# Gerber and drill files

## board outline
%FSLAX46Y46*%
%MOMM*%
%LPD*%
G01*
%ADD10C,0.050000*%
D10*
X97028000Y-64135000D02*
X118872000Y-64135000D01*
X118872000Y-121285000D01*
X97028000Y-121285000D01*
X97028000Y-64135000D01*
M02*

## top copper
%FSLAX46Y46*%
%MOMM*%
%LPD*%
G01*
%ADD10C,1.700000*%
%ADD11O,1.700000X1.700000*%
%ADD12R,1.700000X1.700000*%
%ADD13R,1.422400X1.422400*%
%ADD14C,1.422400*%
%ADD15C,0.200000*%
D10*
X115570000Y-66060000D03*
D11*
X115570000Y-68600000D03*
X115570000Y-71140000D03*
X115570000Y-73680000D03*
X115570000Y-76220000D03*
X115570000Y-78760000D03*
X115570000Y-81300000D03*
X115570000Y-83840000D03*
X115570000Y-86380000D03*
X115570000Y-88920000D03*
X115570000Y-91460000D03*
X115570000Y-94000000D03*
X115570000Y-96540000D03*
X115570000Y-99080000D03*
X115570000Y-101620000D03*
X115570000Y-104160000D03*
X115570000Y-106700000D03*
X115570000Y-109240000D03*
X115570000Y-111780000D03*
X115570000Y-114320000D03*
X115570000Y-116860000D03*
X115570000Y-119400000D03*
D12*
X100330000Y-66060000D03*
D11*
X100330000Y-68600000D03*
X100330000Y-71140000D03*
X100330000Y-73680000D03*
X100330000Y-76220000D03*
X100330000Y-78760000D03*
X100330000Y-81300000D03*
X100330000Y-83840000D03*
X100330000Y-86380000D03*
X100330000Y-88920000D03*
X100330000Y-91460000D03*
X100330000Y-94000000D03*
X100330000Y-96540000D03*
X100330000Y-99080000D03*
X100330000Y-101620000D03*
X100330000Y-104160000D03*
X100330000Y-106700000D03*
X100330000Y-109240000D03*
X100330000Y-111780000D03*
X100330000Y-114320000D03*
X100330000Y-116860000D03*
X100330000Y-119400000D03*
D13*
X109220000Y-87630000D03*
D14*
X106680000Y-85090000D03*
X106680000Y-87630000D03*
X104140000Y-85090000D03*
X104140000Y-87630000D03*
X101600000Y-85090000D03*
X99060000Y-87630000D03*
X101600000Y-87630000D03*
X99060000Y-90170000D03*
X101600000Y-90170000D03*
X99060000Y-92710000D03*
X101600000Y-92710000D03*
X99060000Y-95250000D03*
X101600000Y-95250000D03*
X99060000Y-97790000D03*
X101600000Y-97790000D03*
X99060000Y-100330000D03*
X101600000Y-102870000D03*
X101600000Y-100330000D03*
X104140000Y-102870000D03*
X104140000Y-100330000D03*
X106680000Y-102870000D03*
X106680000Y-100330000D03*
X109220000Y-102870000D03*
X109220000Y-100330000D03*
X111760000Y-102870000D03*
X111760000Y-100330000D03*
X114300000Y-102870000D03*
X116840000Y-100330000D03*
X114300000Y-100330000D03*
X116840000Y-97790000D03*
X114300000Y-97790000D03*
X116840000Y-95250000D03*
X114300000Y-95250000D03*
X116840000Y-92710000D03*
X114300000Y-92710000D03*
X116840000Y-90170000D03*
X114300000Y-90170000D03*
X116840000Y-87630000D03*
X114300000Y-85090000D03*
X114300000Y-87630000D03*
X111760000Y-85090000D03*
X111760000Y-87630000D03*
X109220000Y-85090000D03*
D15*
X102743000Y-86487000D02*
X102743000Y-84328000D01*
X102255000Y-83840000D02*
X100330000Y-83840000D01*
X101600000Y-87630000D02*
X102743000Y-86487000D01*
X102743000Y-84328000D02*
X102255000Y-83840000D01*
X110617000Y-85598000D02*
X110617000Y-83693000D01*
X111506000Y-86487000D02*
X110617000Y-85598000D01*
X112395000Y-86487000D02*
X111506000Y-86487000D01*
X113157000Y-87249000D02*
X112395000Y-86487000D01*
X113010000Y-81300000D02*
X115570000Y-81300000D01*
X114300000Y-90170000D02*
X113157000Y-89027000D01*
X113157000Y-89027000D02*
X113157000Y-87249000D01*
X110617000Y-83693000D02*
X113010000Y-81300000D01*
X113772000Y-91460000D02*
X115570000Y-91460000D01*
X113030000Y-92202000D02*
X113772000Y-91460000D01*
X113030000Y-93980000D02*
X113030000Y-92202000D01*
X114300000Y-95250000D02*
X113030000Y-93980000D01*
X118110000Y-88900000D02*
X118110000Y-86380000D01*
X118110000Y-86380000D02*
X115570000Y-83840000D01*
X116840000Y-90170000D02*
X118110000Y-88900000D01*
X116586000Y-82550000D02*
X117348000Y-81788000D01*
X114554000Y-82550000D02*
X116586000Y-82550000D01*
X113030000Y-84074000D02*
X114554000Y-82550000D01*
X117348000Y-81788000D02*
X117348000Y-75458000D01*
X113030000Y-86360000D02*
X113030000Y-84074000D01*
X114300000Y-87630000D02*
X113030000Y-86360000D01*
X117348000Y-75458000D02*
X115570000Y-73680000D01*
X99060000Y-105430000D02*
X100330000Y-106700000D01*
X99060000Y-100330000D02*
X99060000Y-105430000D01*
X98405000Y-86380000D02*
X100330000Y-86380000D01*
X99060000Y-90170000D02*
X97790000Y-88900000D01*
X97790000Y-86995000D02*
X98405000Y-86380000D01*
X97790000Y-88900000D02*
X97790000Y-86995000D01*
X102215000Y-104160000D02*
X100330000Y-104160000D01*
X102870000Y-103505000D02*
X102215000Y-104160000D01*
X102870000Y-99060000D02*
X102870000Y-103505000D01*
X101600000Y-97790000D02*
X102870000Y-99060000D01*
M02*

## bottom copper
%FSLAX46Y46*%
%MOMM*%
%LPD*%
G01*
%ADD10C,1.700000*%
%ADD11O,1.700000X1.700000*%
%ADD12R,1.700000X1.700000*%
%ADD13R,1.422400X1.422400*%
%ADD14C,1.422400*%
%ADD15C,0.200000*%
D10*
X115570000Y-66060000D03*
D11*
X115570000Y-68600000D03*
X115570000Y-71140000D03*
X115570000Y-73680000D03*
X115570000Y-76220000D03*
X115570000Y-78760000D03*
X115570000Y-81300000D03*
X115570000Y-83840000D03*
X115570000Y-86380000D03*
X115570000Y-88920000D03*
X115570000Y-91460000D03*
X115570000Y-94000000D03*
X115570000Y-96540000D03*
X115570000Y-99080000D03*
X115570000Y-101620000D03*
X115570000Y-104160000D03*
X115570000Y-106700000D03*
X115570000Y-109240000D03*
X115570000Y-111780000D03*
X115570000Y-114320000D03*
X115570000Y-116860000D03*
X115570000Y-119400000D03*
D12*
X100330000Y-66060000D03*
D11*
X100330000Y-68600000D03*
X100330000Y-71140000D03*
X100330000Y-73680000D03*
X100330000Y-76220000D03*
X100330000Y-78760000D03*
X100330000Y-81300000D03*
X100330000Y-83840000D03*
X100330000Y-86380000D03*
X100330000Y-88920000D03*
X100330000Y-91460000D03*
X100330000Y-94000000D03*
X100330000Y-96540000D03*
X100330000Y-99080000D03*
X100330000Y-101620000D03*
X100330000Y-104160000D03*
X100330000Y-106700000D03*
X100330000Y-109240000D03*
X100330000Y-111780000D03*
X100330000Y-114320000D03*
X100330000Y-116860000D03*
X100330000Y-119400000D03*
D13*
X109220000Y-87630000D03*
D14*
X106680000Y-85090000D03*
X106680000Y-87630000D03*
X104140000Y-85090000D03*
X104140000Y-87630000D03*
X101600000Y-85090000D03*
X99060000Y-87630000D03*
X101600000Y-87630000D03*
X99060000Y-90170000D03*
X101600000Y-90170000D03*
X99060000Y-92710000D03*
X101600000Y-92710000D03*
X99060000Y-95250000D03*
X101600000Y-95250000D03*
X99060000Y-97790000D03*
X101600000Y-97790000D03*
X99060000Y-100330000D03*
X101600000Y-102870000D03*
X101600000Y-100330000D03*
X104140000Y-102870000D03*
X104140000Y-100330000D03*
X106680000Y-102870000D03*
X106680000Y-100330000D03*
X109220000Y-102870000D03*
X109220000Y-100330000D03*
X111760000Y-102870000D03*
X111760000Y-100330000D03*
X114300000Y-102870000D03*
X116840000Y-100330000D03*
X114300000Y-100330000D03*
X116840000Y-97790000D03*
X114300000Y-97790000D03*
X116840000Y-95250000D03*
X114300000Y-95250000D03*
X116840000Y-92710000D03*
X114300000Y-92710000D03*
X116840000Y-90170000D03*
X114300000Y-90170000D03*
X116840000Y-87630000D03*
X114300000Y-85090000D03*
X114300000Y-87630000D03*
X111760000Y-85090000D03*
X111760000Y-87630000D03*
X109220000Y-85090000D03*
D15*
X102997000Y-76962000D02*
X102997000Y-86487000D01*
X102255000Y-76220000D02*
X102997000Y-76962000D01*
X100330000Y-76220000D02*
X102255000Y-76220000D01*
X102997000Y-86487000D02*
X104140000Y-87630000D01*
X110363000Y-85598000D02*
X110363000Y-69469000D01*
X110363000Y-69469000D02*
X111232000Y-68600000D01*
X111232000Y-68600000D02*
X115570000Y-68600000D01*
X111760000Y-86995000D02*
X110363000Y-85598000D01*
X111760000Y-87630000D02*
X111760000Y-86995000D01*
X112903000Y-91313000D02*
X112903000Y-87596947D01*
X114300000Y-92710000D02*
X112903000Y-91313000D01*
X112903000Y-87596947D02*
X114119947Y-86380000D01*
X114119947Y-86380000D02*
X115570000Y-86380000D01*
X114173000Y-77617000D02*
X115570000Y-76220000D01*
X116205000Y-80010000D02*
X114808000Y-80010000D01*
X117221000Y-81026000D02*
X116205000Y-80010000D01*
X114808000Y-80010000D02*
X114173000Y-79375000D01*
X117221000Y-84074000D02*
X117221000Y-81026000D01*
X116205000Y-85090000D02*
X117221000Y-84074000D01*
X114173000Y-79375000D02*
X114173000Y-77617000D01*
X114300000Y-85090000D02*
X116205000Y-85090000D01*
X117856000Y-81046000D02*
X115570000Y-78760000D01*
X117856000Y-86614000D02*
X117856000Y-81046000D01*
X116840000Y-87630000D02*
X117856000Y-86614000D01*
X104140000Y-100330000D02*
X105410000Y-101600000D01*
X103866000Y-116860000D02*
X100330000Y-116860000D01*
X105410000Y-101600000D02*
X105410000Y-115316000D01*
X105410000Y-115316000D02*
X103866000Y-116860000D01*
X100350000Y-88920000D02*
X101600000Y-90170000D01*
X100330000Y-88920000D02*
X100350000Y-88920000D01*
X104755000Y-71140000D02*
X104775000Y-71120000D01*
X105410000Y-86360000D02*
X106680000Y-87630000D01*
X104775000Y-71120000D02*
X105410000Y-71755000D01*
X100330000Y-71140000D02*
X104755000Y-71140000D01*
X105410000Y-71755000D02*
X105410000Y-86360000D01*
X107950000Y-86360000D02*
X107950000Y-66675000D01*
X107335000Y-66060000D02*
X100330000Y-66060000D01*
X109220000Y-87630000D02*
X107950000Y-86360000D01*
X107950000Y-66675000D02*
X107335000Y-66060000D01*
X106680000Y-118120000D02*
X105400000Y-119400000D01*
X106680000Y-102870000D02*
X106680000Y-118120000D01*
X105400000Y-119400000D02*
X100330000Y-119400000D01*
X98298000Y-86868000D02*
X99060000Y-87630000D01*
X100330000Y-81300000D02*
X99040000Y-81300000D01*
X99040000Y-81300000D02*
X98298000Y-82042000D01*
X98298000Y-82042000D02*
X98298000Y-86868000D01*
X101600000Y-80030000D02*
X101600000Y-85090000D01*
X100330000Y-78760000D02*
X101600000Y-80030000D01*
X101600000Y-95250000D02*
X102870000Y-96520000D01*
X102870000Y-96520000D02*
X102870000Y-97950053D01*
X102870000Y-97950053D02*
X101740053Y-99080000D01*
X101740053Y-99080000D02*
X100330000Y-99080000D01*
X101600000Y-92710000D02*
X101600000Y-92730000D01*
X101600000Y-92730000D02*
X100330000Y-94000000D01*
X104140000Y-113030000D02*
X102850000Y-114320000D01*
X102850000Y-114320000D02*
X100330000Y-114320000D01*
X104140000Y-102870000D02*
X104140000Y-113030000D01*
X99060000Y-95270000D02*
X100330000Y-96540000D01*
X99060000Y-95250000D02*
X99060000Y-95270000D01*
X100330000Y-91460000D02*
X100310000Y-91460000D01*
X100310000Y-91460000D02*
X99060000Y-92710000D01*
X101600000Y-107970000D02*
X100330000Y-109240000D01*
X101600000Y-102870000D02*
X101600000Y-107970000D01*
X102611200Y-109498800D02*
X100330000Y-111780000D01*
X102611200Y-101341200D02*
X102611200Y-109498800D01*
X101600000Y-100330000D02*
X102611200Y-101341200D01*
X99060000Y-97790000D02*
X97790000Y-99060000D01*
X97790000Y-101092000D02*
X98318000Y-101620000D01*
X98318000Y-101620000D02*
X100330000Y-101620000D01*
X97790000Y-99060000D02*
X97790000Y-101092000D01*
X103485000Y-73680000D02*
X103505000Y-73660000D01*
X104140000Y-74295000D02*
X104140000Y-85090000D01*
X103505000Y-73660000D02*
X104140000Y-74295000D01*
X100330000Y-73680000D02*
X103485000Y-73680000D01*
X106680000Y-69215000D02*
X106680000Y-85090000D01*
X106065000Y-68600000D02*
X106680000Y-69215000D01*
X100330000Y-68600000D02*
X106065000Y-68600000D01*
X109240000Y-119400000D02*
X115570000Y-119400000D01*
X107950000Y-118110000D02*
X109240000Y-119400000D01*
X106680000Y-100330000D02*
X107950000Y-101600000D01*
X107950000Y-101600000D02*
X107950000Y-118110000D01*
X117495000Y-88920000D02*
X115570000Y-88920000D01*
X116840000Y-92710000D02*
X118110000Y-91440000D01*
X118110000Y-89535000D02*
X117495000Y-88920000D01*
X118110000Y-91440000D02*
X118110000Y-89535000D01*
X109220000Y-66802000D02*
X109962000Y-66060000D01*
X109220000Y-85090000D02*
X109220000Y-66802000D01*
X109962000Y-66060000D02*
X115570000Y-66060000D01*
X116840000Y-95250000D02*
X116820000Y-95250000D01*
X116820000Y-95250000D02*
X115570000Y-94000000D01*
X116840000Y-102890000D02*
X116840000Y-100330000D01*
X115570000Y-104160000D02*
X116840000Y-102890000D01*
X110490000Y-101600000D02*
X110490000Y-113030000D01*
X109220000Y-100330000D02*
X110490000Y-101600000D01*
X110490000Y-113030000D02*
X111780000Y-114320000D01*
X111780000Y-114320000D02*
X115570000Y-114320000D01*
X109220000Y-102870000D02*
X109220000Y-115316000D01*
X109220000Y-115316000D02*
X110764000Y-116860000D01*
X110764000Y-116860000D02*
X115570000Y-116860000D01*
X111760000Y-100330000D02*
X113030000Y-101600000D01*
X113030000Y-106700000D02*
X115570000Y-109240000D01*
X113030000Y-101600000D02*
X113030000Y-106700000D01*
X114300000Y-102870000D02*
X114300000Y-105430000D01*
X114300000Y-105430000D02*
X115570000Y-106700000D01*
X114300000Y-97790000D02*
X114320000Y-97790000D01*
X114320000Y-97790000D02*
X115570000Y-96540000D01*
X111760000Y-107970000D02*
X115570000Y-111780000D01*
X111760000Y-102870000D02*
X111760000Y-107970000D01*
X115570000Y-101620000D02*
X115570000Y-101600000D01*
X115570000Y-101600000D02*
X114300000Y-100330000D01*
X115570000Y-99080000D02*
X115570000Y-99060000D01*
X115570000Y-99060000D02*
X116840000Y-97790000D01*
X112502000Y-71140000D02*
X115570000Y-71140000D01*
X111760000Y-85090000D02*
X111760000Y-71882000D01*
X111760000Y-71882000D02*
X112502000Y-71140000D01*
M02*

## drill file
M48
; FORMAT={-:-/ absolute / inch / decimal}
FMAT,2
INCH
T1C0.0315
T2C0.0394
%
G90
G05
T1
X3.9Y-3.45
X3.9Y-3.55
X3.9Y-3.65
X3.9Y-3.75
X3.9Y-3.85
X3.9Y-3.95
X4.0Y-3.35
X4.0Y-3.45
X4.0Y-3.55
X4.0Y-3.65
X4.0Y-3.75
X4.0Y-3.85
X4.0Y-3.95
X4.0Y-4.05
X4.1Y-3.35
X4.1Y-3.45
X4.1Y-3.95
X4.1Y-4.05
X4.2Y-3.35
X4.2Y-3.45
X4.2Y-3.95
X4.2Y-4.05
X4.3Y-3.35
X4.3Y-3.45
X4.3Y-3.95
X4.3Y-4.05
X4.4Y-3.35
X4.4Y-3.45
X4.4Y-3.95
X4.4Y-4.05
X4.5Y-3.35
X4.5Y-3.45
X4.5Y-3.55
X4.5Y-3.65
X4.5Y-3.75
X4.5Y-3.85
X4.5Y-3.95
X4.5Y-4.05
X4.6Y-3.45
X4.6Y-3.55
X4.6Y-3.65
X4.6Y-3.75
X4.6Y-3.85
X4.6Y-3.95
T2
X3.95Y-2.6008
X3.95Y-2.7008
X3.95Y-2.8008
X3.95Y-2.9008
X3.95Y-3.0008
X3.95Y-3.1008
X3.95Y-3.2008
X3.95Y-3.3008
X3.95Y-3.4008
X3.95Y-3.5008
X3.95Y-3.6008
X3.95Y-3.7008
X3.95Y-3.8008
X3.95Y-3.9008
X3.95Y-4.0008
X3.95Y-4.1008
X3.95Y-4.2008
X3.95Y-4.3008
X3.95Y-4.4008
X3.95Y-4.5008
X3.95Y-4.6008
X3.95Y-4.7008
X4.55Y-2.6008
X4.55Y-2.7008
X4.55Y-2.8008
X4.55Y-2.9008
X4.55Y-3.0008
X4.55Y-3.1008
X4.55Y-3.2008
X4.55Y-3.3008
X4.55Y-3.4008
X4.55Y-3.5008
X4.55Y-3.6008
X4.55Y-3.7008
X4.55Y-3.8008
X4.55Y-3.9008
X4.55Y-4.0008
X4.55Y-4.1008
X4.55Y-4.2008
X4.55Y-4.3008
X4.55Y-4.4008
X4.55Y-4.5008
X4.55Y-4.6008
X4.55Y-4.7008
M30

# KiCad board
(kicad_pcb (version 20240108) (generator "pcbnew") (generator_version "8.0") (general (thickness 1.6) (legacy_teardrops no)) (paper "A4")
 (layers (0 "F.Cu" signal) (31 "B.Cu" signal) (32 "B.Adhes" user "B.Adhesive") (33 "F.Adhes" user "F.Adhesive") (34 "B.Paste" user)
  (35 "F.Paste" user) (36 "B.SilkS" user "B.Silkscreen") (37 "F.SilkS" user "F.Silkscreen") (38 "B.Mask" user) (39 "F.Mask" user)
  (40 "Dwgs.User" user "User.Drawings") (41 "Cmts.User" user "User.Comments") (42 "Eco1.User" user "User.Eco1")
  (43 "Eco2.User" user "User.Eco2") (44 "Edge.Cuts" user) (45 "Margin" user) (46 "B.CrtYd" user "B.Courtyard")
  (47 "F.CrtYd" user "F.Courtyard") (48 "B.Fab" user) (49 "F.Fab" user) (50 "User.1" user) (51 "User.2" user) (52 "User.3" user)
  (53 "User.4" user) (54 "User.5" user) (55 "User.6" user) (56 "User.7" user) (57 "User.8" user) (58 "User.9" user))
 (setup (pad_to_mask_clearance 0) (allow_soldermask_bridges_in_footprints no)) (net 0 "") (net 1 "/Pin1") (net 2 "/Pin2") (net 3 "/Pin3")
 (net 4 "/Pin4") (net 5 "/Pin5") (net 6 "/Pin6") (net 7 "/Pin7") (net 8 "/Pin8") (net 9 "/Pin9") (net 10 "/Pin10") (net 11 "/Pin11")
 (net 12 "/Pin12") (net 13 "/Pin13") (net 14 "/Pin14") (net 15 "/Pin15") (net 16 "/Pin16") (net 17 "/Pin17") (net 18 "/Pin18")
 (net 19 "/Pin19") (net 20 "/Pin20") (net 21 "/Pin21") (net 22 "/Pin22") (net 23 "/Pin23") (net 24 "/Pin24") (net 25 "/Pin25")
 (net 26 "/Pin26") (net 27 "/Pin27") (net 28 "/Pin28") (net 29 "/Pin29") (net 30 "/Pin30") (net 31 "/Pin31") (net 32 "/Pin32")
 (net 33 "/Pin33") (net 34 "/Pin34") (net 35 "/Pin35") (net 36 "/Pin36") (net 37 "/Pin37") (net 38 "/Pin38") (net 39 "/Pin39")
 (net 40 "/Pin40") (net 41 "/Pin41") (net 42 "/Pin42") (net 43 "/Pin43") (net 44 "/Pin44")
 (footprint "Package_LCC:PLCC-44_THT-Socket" (layer "F.Cu") (at 109.22 87.63)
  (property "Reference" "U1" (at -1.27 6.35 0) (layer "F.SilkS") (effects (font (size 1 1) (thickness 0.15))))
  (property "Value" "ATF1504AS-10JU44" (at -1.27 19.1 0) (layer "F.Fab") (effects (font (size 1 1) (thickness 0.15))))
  (pad "1" thru_hole rect (at 0 0) (size 1.4224 1.4224) (drill 0.8) (layers "*.Cu" "*.Mask") (remove_unused_layers no) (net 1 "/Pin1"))
  (pad "2" thru_hole circle (at -2.54 -2.54) (size 1.4224 1.4224) (drill 0.8) (layers "*.Cu" "*.Mask") (remove_unused_layers no)
   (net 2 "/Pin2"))
  (pad "3" thru_hole circle (at -2.54 0) (size 1.4224 1.4224) (drill 0.8) (layers "*.Cu" "*.Mask") (remove_unused_layers no) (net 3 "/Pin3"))
  (pad "4" thru_hole circle (at -5.08 -2.54) (size 1.4224 1.4224) (drill 0.8) (layers "*.Cu" "*.Mask") (remove_unused_layers no)
   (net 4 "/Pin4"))
  (pad "5" thru_hole circle (at -5.08 0) (size 1.4224 1.4224) (drill 0.8) (layers "*.Cu" "*.Mask") (remove_unused_layers no) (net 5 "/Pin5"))
  (pad "6" thru_hole circle (at -7.62 -2.54) (size 1.4224 1.4224) (drill 0.8) (layers "*.Cu" "*.Mask") (remove_unused_layers no)
   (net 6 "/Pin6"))
  (pad "7" thru_hole circle (at -10.16 0) (size 1.4224 1.4224) (drill 0.8) (layers "*.Cu" "*.Mask") (remove_unused_layers no)
   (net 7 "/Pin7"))
  (pad "8" thru_hole circle (at -7.62 0) (size 1.4224 1.4224) (drill 0.8) (layers "*.Cu" "*.Mask") (remove_unused_layers no) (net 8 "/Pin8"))
  (pad "9" thru_hole circle (at -10.16 2.54) (size 1.4224 1.4224) (drill 0.8) (layers "*.Cu" "*.Mask") (remove_unused_layers no)
   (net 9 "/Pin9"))
  (pad "10" thru_hole circle (at -7.62 2.54) (size 1.4224 1.4224) (drill 0.8) (layers "*.Cu" "*.Mask") (remove_unused_layers no)
   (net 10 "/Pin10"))
  (pad "11" thru_hole circle (at -10.16 5.08) (size 1.4224 1.4224) (drill 0.8) (layers "*.Cu" "*.Mask") (remove_unused_layers no)
   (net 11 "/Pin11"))
  (pad "12" thru_hole circle (at -7.62 5.08) (size 1.4224 1.4224) (drill 0.8) (layers "*.Cu" "*.Mask") (remove_unused_layers no)
   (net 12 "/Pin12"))
  (pad "13" thru_hole circle (at -10.16 7.62) (size 1.4224 1.4224) (drill 0.8) (layers "*.Cu" "*.Mask") (remove_unused_layers no)
   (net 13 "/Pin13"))
  (pad "14" thru_hole circle (at -7.62 7.62) (size 1.4224 1.4224) (drill 0.8) (layers "*.Cu" "*.Mask") (remove_unused_layers no)
   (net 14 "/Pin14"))
  (pad "15" thru_hole circle (at -10.16 10.16) (size 1.4224 1.4224) (drill 0.8) (layers "*.Cu" "*.Mask") (remove_unused_layers no)
   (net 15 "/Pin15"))
  (pad "16" thru_hole circle (at -7.62 10.16) (size 1.4224 1.4224) (drill 0.8) (layers "*.Cu" "*.Mask") (remove_unused_layers no)
   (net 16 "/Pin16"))
  (pad "17" thru_hole circle (at -10.16 12.7) (size 1.4224 1.4224) (drill 0.8) (layers "*.Cu" "*.Mask") (remove_unused_layers no)
   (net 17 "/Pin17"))
  (pad "18" thru_hole circle (at -7.62 15.24) (size 1.4224 1.4224) (drill 0.8) (layers "*.Cu" "*.Mask") (remove_unused_layers no)
   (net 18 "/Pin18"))
  (pad "19" thru_hole circle (at -7.62 12.7) (size 1.4224 1.4224) (drill 0.8) (layers "*.Cu" "*.Mask") (remove_unused_layers no)
   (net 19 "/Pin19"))
  (pad "20" thru_hole circle (at -5.08 15.24) (size 1.4224 1.4224) (drill 0.8) (layers "*.Cu" "*.Mask") (remove_unused_layers no)
   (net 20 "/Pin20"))
  (pad "21" thru_hole circle (at -5.08 12.7) (size 1.4224 1.4224) (drill 0.8) (layers "*.Cu" "*.Mask") (remove_unused_layers no)
   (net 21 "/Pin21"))
  (pad "22" thru_hole circle (at -2.54 15.24) (size 1.4224 1.4224) (drill 0.8) (layers "*.Cu" "*.Mask") (remove_unused_layers no)
   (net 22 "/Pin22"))
  (pad "23" thru_hole circle (at -2.54 12.7) (size 1.4224 1.4224) (drill 0.8) (layers "*.Cu" "*.Mask") (remove_unused_layers no)
   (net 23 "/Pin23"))
  (pad "24" thru_hole circle (at 0 15.24) (size 1.4224 1.4224) (drill 0.8) (layers "*.Cu" "*.Mask") (remove_unused_layers no)
   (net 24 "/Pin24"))
  (pad "25" thru_hole circle (at 0 12.7) (size 1.4224 1.4224) (drill 0.8) (layers "*.Cu" "*.Mask") (remove_unused_layers no)
   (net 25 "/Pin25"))
  (pad "26" thru_hole circle (at 2.54 15.24) (size 1.4224 1.4224) (drill 0.8) (layers "*.Cu" "*.Mask") (remove_unused_layers no)
   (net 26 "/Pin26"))
  (pad "27" thru_hole circle (at 2.54 12.7) (size 1.4224 1.4224) (drill 0.8) (layers "*.Cu" "*.Mask") (remove_unused_layers no)
   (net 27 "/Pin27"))
  (pad "28" thru_hole circle (at 5.08 15.24) (size 1.4224 1.4224) (drill 0.8) (layers "*.Cu" "*.Mask") (remove_unused_layers no)
   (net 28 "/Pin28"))
  (pad "29" thru_hole circle (at 7.62 12.7) (size 1.4224 1.4224) (drill 0.8) (layers "*.Cu" "*.Mask") (remove_unused_layers no)
   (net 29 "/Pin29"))
  (pad "30" thru_hole circle (at 5.08 12.7) (size 1.4224 1.4224) (drill 0.8) (layers "*.Cu" "*.Mask") (remove_unused_layers no)
   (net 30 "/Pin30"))
  (pad "31" thru_hole circle (at 7.62 10.16) (size 1.4224 1.4224) (drill 0.8) (layers "*.Cu" "*.Mask") (remove_unused_layers no)
   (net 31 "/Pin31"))
  (pad "32" thru_hole circle (at 5.08 10.16) (size 1.4224 1.4224) (drill 0.8) (layers "*.Cu" "*.Mask") (remove_unused_layers no)
   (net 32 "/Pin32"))
  (pad "33" thru_hole circle (at 7.62 7.62) (size 1.4224 1.4224) (drill 0.8) (layers "*.Cu" "*.Mask") (remove_unused_layers no)
   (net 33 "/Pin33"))
  (pad "34" thru_hole circle (at 5.08 7.62) (size 1.4224 1.4224) (drill 0.8) (layers "*.Cu" "*.Mask") (remove_unused_layers no)
   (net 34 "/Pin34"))
  (pad "35" thru_hole circle (at 7.62 5.08) (size 1.4224 1.4224) (drill 0.8) (layers "*.Cu" "*.Mask") (remove_unused_layers no)
   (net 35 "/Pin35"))
  (pad "36" thru_hole circle (at 5.08 5.08) (size 1.4224 1.4224) (drill 0.8) (layers "*.Cu" "*.Mask") (remove_unused_layers no)
   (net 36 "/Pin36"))
  (pad "37" thru_hole circle (at 7.62 2.54) (size 1.4224 1.4224) (drill 0.8) (layers "*.Cu" "*.Mask") (remove_unused_layers no)
   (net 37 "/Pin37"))
  (pad "38" thru_hole circle (at 5.08 2.54) (size 1.4224 1.4224) (drill 0.8) (layers "*.Cu" "*.Mask") (remove_unused_layers no)
   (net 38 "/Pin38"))
  (pad "39" thru_hole circle (at 7.62 0) (size 1.4224 1.4224) (drill 0.8) (layers "*.Cu" "*.Mask") (remove_unused_layers no)
   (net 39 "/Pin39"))
  (pad "40" thru_hole circle (at 5.08 -2.54) (size 1.4224 1.4224) (drill 0.8) (layers "*.Cu" "*.Mask") (remove_unused_layers no)
   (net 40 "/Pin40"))
  (pad "41" thru_hole circle (at 5.08 0) (size 1.4224 1.4224) (drill 0.8) (layers "*.Cu" "*.Mask") (remove_unused_layers no)
   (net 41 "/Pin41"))
  (pad "42" thru_hole circle (at 2.54 -2.54) (size 1.4224 1.4224) (drill 0.8) (layers "*.Cu" "*.Mask") (remove_unused_layers no)
   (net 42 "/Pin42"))
  (pad "43" thru_hole circle (at 2.54 0) (size 1.4224 1.4224) (drill 0.8) (layers "*.Cu" "*.Mask") (remove_unused_layers no)
   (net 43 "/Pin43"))
  (pad "44" thru_hole circle (at 0 -2.54) (size 1.4224 1.4224) (drill 0.8) (layers "*.Cu" "*.Mask") (remove_unused_layers no)
   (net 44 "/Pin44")))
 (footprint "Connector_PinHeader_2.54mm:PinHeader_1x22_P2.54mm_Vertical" (layer "B.Cu") (at 115.57 66.06 180)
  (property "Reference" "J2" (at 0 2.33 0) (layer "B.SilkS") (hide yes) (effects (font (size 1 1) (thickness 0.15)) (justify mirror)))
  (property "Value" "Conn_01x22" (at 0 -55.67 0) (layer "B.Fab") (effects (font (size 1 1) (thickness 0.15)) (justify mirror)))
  (pad "1" thru_hole circle (at 0 0 180) (size 1.7 1.7) (drill 1) (layers "*.Cu" "*.Mask") (remove_unused_layers no) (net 44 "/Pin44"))
  (pad "2" thru_hole oval (at 0 -2.54 180) (size 1.7 1.7) (drill 1) (layers "*.Cu" "*.Mask") (remove_unused_layers no) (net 43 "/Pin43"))
  (pad "3" thru_hole oval (at 0 -5.08 180) (size 1.7 1.7) (drill 1) (layers "*.Cu" "*.Mask") (remove_unused_layers no) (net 42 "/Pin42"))
  (pad "4" thru_hole oval (at 0 -7.62 180) (size 1.7 1.7) (drill 1) (layers "*.Cu" "*.Mask") (remove_unused_layers no) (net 41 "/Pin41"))
  (pad "5" thru_hole oval (at 0 -10.16 180) (size 1.7 1.7) (drill 1) (layers "*.Cu" "*.Mask") (remove_unused_layers no) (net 40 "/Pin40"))
  (pad "6" thru_hole oval (at 0 -12.7 180) (size 1.7 1.7) (drill 1) (layers "*.Cu" "*.Mask") (remove_unused_layers no) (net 39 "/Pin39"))
  (pad "7" thru_hole oval (at 0 -15.24 180) (size 1.7 1.7) (drill 1) (layers "*.Cu" "*.Mask") (remove_unused_layers no) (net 38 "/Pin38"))
  (pad "8" thru_hole oval (at 0 -17.78 180) (size 1.7 1.7) (drill 1) (layers "*.Cu" "*.Mask") (remove_unused_layers no) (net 37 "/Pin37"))
  (pad "9" thru_hole oval (at 0 -20.32 180) (size 1.7 1.7) (drill 1) (layers "*.Cu" "*.Mask") (remove_unused_layers no) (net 36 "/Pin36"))
  (pad "10" thru_hole oval (at 0 -22.86 180) (size 1.7 1.7) (drill 1) (layers "*.Cu" "*.Mask") (remove_unused_layers no) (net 35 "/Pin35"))
  (pad "11" thru_hole oval (at 0 -25.4 180) (size 1.7 1.7) (drill 1) (layers "*.Cu" "*.Mask") (remove_unused_layers no) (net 34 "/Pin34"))
  (pad "12" thru_hole oval (at 0 -27.94 180) (size 1.7 1.7) (drill 1) (layers "*.Cu" "*.Mask") (remove_unused_layers no) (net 33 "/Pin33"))
  (pad "13" thru_hole oval (at 0 -30.48 180) (size 1.7 1.7) (drill 1) (layers "*.Cu" "*.Mask") (remove_unused_layers no) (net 32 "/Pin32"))
  (pad "14" thru_hole oval (at 0 -33.02 180) (size 1.7 1.7) (drill 1) (layers "*.Cu" "*.Mask") (remove_unused_layers no) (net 31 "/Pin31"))
  (pad "15" thru_hole oval (at 0 -35.56 180) (size 1.7 1.7) (drill 1) (layers "*.Cu" "*.Mask") (remove_unused_layers no) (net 30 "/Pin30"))
  (pad "16" thru_hole oval (at 0 -38.1 180) (size 1.7 1.7) (drill 1) (layers "*.Cu" "*.Mask") (remove_unused_layers no) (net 29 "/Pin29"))
  (pad "17" thru_hole oval (at 0 -40.64 180) (size 1.7 1.7) (drill 1) (layers "*.Cu" "*.Mask") (remove_unused_layers no) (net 28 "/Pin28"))
  (pad "18" thru_hole oval (at 0 -43.18 180) (size 1.7 1.7) (drill 1) (layers "*.Cu" "*.Mask") (remove_unused_layers no) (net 27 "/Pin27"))
  (pad "19" thru_hole oval (at 0 -45.72 180) (size 1.7 1.7) (drill 1) (layers "*.Cu" "*.Mask") (remove_unused_layers no) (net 26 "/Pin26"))
  (pad "20" thru_hole oval (at 0 -48.26 180) (size 1.7 1.7) (drill 1) (layers "*.Cu" "*.Mask") (remove_unused_layers no) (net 25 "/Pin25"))
  (pad "21" thru_hole oval (at 0 -50.8 180) (size 1.7 1.7) (drill 1) (layers "*.Cu" "*.Mask") (remove_unused_layers no) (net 24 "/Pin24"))
  (pad "22" thru_hole oval (at 0 -53.34 180) (size 1.7 1.7) (drill 1) (layers "*.Cu" "*.Mask") (remove_unused_layers no) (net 23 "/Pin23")))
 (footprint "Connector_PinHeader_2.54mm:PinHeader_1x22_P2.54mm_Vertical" (layer "B.Cu") (at 100.33 66.06 180)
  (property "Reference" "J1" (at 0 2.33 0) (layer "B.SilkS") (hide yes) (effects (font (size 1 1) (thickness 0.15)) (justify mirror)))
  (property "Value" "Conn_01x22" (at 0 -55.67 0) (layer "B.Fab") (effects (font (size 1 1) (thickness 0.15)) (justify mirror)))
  (pad "1" thru_hole rect (at 0 0 180) (size 1.7 1.7) (drill 1) (layers "*.Cu" "*.Mask") (remove_unused_layers no) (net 1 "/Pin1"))
  (pad "2" thru_hole oval (at 0 -2.54 180) (size 1.7 1.7) (drill 1) (layers "*.Cu" "*.Mask") (remove_unused_layers no) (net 2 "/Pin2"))
  (pad "3" thru_hole oval (at 0 -5.08 180) (size 1.7 1.7) (drill 1) (layers "*.Cu" "*.Mask") (remove_unused_layers no) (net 3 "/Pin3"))
  (pad "4" thru_hole oval (at 0 -7.62 180) (size 1.7 1.7) (drill 1) (layers "*.Cu" "*.Mask") (remove_unused_layers no) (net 4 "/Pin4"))
  (pad "5" thru_hole oval (at 0 -10.16 180) (size 1.7 1.7) (drill 1) (layers "*.Cu" "*.Mask") (remove_unused_layers no) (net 5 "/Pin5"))
  (pad "6" thru_hole oval (at 0 -12.7 180) (size 1.7 1.7) (drill 1) (layers "*.Cu" "*.Mask") (remove_unused_layers no) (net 6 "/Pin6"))
  (pad "7" thru_hole oval (at 0 -15.24 180) (size 1.7 1.7) (drill 1) (layers "*.Cu" "*.Mask") (remove_unused_layers no) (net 7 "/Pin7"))
  (pad "8" thru_hole oval (at 0 -17.78 180) (size 1.7 1.7) (drill 1) (layers "*.Cu" "*.Mask") (remove_unused_layers no) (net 8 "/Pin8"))
  (pad "9" thru_hole oval (at 0 -20.32 180) (size 1.7 1.7) (drill 1) (layers "*.Cu" "*.Mask") (remove_unused_layers no) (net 9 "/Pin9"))
  (pad "10" thru_hole oval (at 0 -22.86 180) (size 1.7 1.7) (drill 1) (layers "*.Cu" "*.Mask") (remove_unused_layers no) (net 10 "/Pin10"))
  (pad "11" thru_hole oval (at 0 -25.4 180) (size 1.7 1.7) (drill 1) (layers "*.Cu" "*.Mask") (remove_unused_layers no) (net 11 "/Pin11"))
  (pad "12" thru_hole oval (at 0 -27.94 180) (size 1.7 1.7) (drill 1) (layers "*.Cu" "*.Mask") (remove_unused_layers no) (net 12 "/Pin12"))
  (pad "13" thru_hole oval (at 0 -30.48 180) (size 1.7 1.7) (drill 1) (layers "*.Cu" "*.Mask") (remove_unused_layers no) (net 13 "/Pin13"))
  (pad "14" thru_hole oval (at 0 -33.02 180) (size 1.7 1.7) (drill 1) (layers "*.Cu" "*.Mask") (remove_unused_layers no) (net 14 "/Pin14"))
  (pad "15" thru_hole oval (at 0 -35.56 180) (size 1.7 1.7) (drill 1) (layers "*.Cu" "*.Mask") (remove_unused_layers no) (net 15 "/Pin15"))
  (pad "16" thru_hole oval (at 0 -38.1 180) (size 1.7 1.7) (drill 1) (layers "*.Cu" "*.Mask") (remove_unused_layers no) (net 16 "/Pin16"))
  (pad "17" thru_hole oval (at 0 -40.64 180) (size 1.7 1.7) (drill 1) (layers "*.Cu" "*.Mask") (remove_unused_layers no) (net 17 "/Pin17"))
  (pad "18" thru_hole oval (at 0 -43.18 180) (size 1.7 1.7) (drill 1) (layers "*.Cu" "*.Mask") (remove_unused_layers no) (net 18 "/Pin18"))
  (pad "19" thru_hole oval (at 0 -45.72 180) (size 1.7 1.7) (drill 1) (layers "*.Cu" "*.Mask") (remove_unused_layers no) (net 19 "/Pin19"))
  (pad "20" thru_hole oval (at 0 -48.26 180) (size 1.7 1.7) (drill 1) (layers "*.Cu" "*.Mask") (remove_unused_layers no) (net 20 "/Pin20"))
  (pad "21" thru_hole oval (at 0 -50.8 180) (size 1.7 1.7) (drill 1) (layers "*.Cu" "*.Mask") (remove_unused_layers no) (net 21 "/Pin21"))
  (pad "22" thru_hole oval (at 0 -53.34 180) (size 1.7 1.7) (drill 1) (layers "*.Cu" "*.Mask") (remove_unused_layers no) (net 22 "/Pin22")))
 (gr_rect (start 97.028 64.135) (end 118.872 121.285) (stroke (width 0.05) (type default)) (fill none) (layer "Edge.Cuts"))
 (segment (start 104.14 100.33) (end 105.41 101.6) (width 0.2) (layer "B.Cu") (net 21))
 (segment (start 103.866 116.86) (end 100.33 116.86) (width 0.2) (layer "B.Cu") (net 21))
 (segment (start 105.41 101.6) (end 105.41 115.316) (width 0.2) (layer "B.Cu") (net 21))
 (segment (start 105.41 115.316) (end 103.866 116.86) (width 0.2) (layer "B.Cu") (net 21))
 (segment (start 100.35 88.92) (end 101.6 90.17) (width 0.2) (layer "B.Cu") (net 10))
 (segment (start 100.33 88.92) (end 100.35 88.92) (width 0.2) (layer "B.Cu") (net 10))
 (segment (start 99.06 105.43) (end 100.33 106.7) (width 0.2) (layer "F.Cu") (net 17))
 (segment (start 99.06 100.33) (end 99.06 105.43) (width 0.2) (layer "F.Cu") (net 17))
 (segment (start 104.755 71.14) (end 104.775 71.12) (width 0.2) (layer "B.Cu") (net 3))
 (segment (start 105.41 86.36) (end 106.68 87.63) (width 0.2) (layer "B.Cu") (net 3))
 (segment (start 104.775 71.12) (end 105.41 71.755) (width 0.2) (layer "B.Cu") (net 3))
 (segment (start 100.33 71.14) (end 104.755 71.14) (width 0.2) (layer "B.Cu") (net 3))
 (segment (start 105.41 71.755) (end 105.41 86.36) (width 0.2) (layer "B.Cu") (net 3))
 (segment (start 107.95 86.36) (end 107.95 66.675) (width 0.2) (layer "B.Cu") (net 1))
 (segment (start 107.335 66.06) (end 100.33 66.06) (width 0.2) (layer "B.Cu") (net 1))
 (segment (start 109.22 87.63) (end 107.95 86.36) (width 0.2) (layer "B.Cu") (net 1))
 (segment (start 107.95 66.675) (end 107.335 66.06) (width 0.2) (layer "B.Cu") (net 1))
 (segment (start 106.68 118.12) (end 105.4 119.4) (width 0.2) (layer "B.Cu") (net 22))
 (segment (start 106.68 102.87) (end 106.68 118.12) (width 0.2) (layer "B.Cu") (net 22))
 (segment (start 105.4 119.4) (end 100.33 119.4) (width 0.2) (layer "B.Cu") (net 22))
 (segment (start 102.743 84.328) (end 102.255 83.84) (width 0.2) (layer "F.Cu") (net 8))
 (segment (start 101.6 87.63) (end 102.743 86.487) (width 0.2) (layer "F.Cu") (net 8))
 (segment (start 102.743 86.487) (end 102.743 84.328) (width 0.2) (layer "F.Cu") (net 8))
 (segment (start 102.255 83.84) (end 100.33 83.84) (width 0.2) (layer "F.Cu") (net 8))
 (segment (start 98.298 86.868) (end 99.06 87.63) (width 0.2) (layer "B.Cu") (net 7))
 (segment (start 100.33 81.3) (end 99.04 81.3) (width 0.2) (layer "B.Cu") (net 7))
 (segment (start 99.04 81.3) (end 98.298 82.042) (width 0.2) (layer "B.Cu") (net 7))
 (segment (start 98.298 82.042) (end 98.298 86.868) (width 0.2) (layer "B.Cu") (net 7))
 (segment (start 101.6 80.03) (end 101.6 85.09) (width 0.2) (layer "B.Cu") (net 6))
 (segment (start 100.33 78.76) (end 101.6 80.03) (width 0.2) (layer "B.Cu") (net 6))
 (segment (start 101.6 95.25) (end 102.87 96.52) (width 0.2) (layer "B.Cu") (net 14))
 (segment (start 102.87 96.52) (end 102.87 97.950053) (width 0.2) (layer "B.Cu") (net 14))
 (segment (start 102.87 97.950053) (end 101.740053 99.08) (width 0.2) (layer "B.Cu") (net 14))
 (segment (start 101.740053 99.08) (end 100.33 99.08) (width 0.2) (layer "B.Cu") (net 14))
 (segment (start 101.6 92.71) (end 101.6 92.73) (width 0.2) (layer "B.Cu") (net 12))
 (segment (start 101.6 92.73) (end 100.33 94) (width 0.2) (layer "B.Cu") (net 12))
 (segment (start 98.405 86.38) (end 100.33 86.38) (width 0.2) (layer "F.Cu") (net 9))
 (segment (start 99.06 90.17) (end 97.79 88.9) (width 0.2) (layer "F.Cu") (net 9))
 (segment (start 97.79 86.995) (end 98.405 86.38) (width 0.2) (layer "F.Cu") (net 9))
 (segment (start 97.79 88.9) (end 97.79 86.995) (width 0.2) (layer "F.Cu") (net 9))
 (segment (start 104.14 113.03) (end 102.85 114.32) (width 0.2) (layer "B.Cu") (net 20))
 (segment (start 102.85 114.32) (end 100.33 114.32) (width 0.2) (layer "B.Cu") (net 20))
 (segment (start 104.14 102.87) (end 104.14 113.03) (width 0.2) (layer "B.Cu") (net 20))
 (segment (start 99.06 95.27) (end 100.33 96.54) (width 0.2) (layer "B.Cu") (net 13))
 (segment (start 99.06 95.25) (end 99.06 95.27) (width 0.2) (layer "B.Cu") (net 13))
 (segment (start 100.33 91.46) (end 100.31 91.46) (width 0.2) (layer "B.Cu") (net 11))
 (segment (start 100.31 91.46) (end 99.06 92.71) (width 0.2) (layer "B.Cu") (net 11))
 (segment (start 100.33 76.22) (end 102.255 76.22) (width 0.2) (layer "B.Cu") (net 5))
 (segment (start 102.997 86.487) (end 104.14 87.63) (width 0.2) (layer "B.Cu") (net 5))
 (segment (start 102.255 76.22) (end 102.997 76.962) (width 0.2) (layer "B.Cu") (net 5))
 (segment (start 102.997 76.962) (end 102.997 86.487) (width 0.2) (layer "B.Cu") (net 5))
 (segment (start 101.6 107.97) (end 100.33 109.24) (width 0.2) (layer "B.Cu") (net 18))
 (segment (start 101.6 102.87) (end 101.6 107.97) (width 0.2) (layer "B.Cu") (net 18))
 (segment (start 102.6112 109.4988) (end 100.33 111.78) (width 0.2) (layer "B.Cu") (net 19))
 (segment (start 102.6112 101.3412) (end 102.6112 109.4988) (width 0.2) (layer "B.Cu") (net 19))
 (segment (start 101.6 100.33) (end 102.6112 101.3412) (width 0.2) (layer "B.Cu") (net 19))
 (segment (start 99.06 97.79) (end 97.79 99.06) (width 0.2) (layer "B.Cu") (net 15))
 (segment (start 97.79 101.092) (end 98.318 101.62) (width 0.2) (layer "B.Cu") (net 15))
 (segment (start 98.318 101.62) (end 100.33 101.62) (width 0.2) (layer "B.Cu") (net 15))
 (segment (start 97.79 99.06) (end 97.79 101.092) (width 0.2) (layer "B.Cu") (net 15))
 (segment (start 102.215 104.16) (end 100.33 104.16) (width 0.2) (layer "F.Cu") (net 16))
 (segment (start 102.87 103.505) (end 102.215 104.16) (width 0.2) (layer "F.Cu") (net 16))
 (segment (start 102.87 99.06) (end 102.87 103.505) (width 0.2) (layer "F.Cu") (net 16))
 (segment (start 101.6 97.79) (end 102.87 99.06) (width 0.2) (layer "F.Cu") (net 16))
 (segment (start 103.485 73.68) (end 103.505 73.66) (width 0.2) (layer "B.Cu") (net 4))
 (segment (start 104.14 74.295) (end 104.14 85.09) (width 0.2) (layer "B.Cu") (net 4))
 (segment (start 103.505 73.66) (end 104.14 74.295) (width 0.2) (layer "B.Cu") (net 4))
 (segment (start 100.33 73.68) (end 103.485 73.68) (width 0.2) (layer "B.Cu") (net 4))
 (segment (start 106.68 69.215) (end 106.68 85.09) (width 0.2) (layer "B.Cu") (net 2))
 (segment (start 106.065 68.6) (end 106.68 69.215) (width 0.2) (layer "B.Cu") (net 2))
 (segment (start 100.33 68.6) (end 106.065 68.6) (width 0.2) (layer "B.Cu") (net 2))
 (segment (start 113.772 91.46) (end 115.57 91.46) (width 0.2) (layer "F.Cu") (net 34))
 (segment (start 113.03 93.98) (end 113.03 92.202) (width 0.2) (layer "F.Cu") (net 34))
 (segment (start 113.03 92.202) (end 113.772 91.46) (width 0.2) (layer "F.Cu") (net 34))
 (segment (start 114.3 95.25) (end 113.03 93.98) (width 0.2) (layer "F.Cu") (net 34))
 (segment (start 113.01 81.3) (end 115.57 81.3) (width 0.2) (layer "F.Cu") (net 38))
 (segment (start 111.506 86.487) (end 110.617 85.598) (width 0.2) (layer "F.Cu") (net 38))
 (segment (start 110.617 85.598) (end 110.617 83.693) (width 0.2) (layer "F.Cu") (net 38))
 (segment (start 113.157 89.027) (end 113.157 87.249) (width 0.2) (layer "F.Cu") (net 38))
 (segment (start 112.395 86.487) (end 111.506 86.487) (width 0.2) (layer "F.Cu") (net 38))
 (segment (start 110.617 83.693) (end 113.01 81.3) (width 0.2) (layer "F.Cu") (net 38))
 (segment (start 114.3 90.17) (end 113.157 89.027) (width 0.2) (layer "F.Cu") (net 38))
 (segment (start 113.157 87.249) (end 112.395 86.487) (width 0.2) (layer "F.Cu") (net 38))
 (segment (start 109.24 119.4) (end 115.57 119.4) (width 0.2) (layer "B.Cu") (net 23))
 (segment (start 107.95 118.11) (end 109.24 119.4) (width 0.2) (layer "B.Cu") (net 23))
 (segment (start 106.68 100.33) (end 107.95 101.6) (width 0.2) (layer "B.Cu") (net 23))
 (segment (start 107.95 101.6) (end 107.95 118.11) (width 0.2) (layer "B.Cu") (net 23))
 (segment (start 117.495 88.92) (end 115.57 88.92) (width 0.2) (layer "B.Cu") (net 35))
 (segment (start 116.84 92.71) (end 118.11 91.44) (width 0.2) (layer "B.Cu") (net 35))
 (segment (start 118.11 89.535) (end 117.495 88.92) (width 0.2) (layer "B.Cu") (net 35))
 (segment (start 118.11 91.44) (end 118.11 89.535) (width 0.2) (layer "B.Cu") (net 35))
 (segment (start 109.22 66.802) (end 109.962 66.06) (width 0.2) (layer "B.Cu") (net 44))
 (segment (start 109.22 85.09) (end 109.22 66.802) (width 0.2) (layer "B.Cu") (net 44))
 (segment (start 109.962 66.06) (end 115.57 66.06) (width 0.2) (layer "B.Cu") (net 44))
 (segment (start 116.84 95.25) (end 116.82 95.25) (width 0.2) (layer "B.Cu") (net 33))
 (segment (start 116.82 95.25) (end 115.57 94) (width 0.2) (layer "B.Cu") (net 33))
 (segment (start 116.205 80.01) (end 114.808 80.01) (width 0.2) (layer "B.Cu") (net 40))
 (segment (start 117.221 81.026) (end 116.205 80.01) (width 0.2) (layer "B.Cu") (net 40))
 (segment (start 116.205 85.09) (end 117.221 84.074) (width 0.2) (layer "B.Cu") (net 40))
 (segment (start 114.808 80.01) (end 114.173 79.375) (width 0.2) (layer "B.Cu") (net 40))
 (segment (start 114.173 77.617) (end 115.57 76.22) (width 0.2) (layer "B.Cu") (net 40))
 (segment (start 114.3 85.09) (end 116.205 85.09) (width 0.2) (layer "B.Cu") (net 40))
 (segment (start 114.173 79.375) (end 114.173 77.617) (width 0.2) (layer "B.Cu") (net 40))
 (segment (start 117.221 84.074) (end 117.221 81.026) (width 0.2) (layer "B.Cu") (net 40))
 (segment (start 116.84 102.89) (end 116.84 100.33) (width 0.2) (layer "B.Cu") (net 29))
 (segment (start 115.57 104.16) (end 116.84 102.89) (width 0.2) (layer "B.Cu") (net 29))
 (segment (start 116.84 90.17) (end 118.11 88.9) (width 0.2) (layer "F.Cu") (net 37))
 (segment (start 118.11 88.9) (end 118.11 86.38) (width 0.2) (layer "F.Cu") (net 37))
 (segment (start 118.11 86.38) (end 115.57 83.84) (width 0.2) (layer "F.Cu") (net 37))
 (segment (start 117.348 81.788) (end 117.348 75.458) (width 0.2) (layer "F.Cu") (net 41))
 (segment (start 114.3 87.63) (end 113.03 86.36) (width 0.2) (layer "F.Cu") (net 41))
 (segment (start 113.03 86.36) (end 113.03 84.074) (width 0.2) (layer "F.Cu") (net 41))
 (segment (start 114.554 82.55) (end 116.586 82.55) (width 0.2) (layer "F.Cu") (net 41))
 (segment (start 116.586 82.55) (end 117.348 81.788) (width 0.2) (layer "F.Cu") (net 41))
 (segment (start 113.03 84.074) (end 114.554 82.55) (width 0.2) (layer "F.Cu") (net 41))
 (segment (start 117.348 75.458) (end 115.57 73.68) (width 0.2) (layer "F.Cu") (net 41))
 (segment (start 110.49 101.6) (end 110.49 113.03) (width 0.2) (layer "B.Cu") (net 25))
 (segment (start 109.22 100.33) (end 110.49 101.6) (width 0.2) (layer "B.Cu") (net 25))
 (segment (start 110.49 113.03) (end 111.78 114.32) (width 0.2) (layer "B.Cu") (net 25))
 (segment (start 111.78 114.32) (end 115.57 114.32) (width 0.2) (layer "B.Cu") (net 25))
 (segment (start 109.22 102.87) (end 109.22 115.316) (width 0.2) (layer "B.Cu") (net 24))
 (segment (start 109.22 115.316) (end 110.764 116.86) (width 0.2) (layer "B.Cu") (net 24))
 (segment (start 110.764 116.86) (end 115.57 116.86) (width 0.2) (layer "B.Cu") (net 24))
 (segment (start 116.84 87.63) (end 117.856 86.614) (width 0.2) (layer "B.Cu") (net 39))
 (segment (start 117.856 86.614) (end 117.856 81.046) (width 0.2) (layer "B.Cu") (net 39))
 (segment (start 117.856 81.046) (end 115.57 78.76) (width 0.2) (layer "B.Cu") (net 39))
 (segment (start 110.363 85.598) (end 110.363 69.469) (width 0.2) (layer "B.Cu") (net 43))
 (segment (start 111.76 87.63) (end 111.76 86.995) (width 0.2) (layer "B.Cu") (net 43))
 (segment (start 111.76 86.995) (end 110.363 85.598) (width 0.2) (layer "B.Cu") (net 43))
 (segment (start 110.363 69.469) (end 111.232 68.6) (width 0.2) (layer "B.Cu") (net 43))
 (segment (start 111.232 68.6) (end 115.57 68.6) (width 0.2) (layer "B.Cu") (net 43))
 (segment (start 111.76 100.33) (end 113.03 101.6) (width 0.2) (layer "B.Cu") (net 27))
 (segment (start 113.03 106.7) (end 115.57 109.24) (width 0.2) (layer "B.Cu") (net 27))
 (segment (start 113.03 101.6) (end 113.03 106.7) (width 0.2) (layer "B.Cu") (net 27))
 (segment (start 114.3 102.87) (end 114.3 105.43) (width 0.2) (layer "B.Cu") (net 28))
 (segment (start 114.3 105.43) (end 115.57 106.7) (width 0.2) (layer "B.Cu") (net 28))
 (segment (start 114.3 97.79) (end 114.32 97.79) (width 0.2) (layer "B.Cu") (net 32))
 (segment (start 114.32 97.79) (end 115.57 96.54) (width 0.2) (layer "B.Cu") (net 32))
 (segment (start 111.76 107.97) (end 115.57 111.78) (width 0.2) (layer "B.Cu") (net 26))
 (segment (start 111.76 102.87) (end 111.76 107.97) (width 0.2) (layer "B.Cu") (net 26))
 (segment (start 115.57 101.62) (end 115.57 101.6) (width 0.2) (layer "B.Cu") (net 30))
 (segment (start 115.57 101.6) (end 114.3 100.33) (width 0.2) (layer "B.Cu") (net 30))
 (segment (start 115.57 99.08) (end 115.57 99.06) (width 0.2) (layer "B.Cu") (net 31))
 (segment (start 115.57 99.06) (end 116.84 97.79) (width 0.2) (layer "B.Cu") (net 31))
 (segment (start 112.903 87.596947) (end 114.119947 86.38) (width 0.2) (layer "B.Cu") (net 36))
 (segment (start 114.3 92.71) (end 112.903 91.313) (width 0.2) (layer "B.Cu") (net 36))
 (segment (start 114.119947 86.38) (end 115.57 86.38) (width 0.2) (layer "B.Cu") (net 36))
 (segment (start 112.903 91.313) (end 112.903 87.596947) (width 0.2) (layer "B.Cu") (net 36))
 (segment (start 112.502 71.14) (end 115.57 71.14) (width 0.2) (layer "B.Cu") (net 42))
 (segment (start 111.76 85.09) (end 111.76 71.882) (width 0.2) (layer "B.Cu") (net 42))
 (segment (start 111.76 71.882) (end 112.502 71.14) (width 0.2) (layer "B.Cu") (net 42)))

